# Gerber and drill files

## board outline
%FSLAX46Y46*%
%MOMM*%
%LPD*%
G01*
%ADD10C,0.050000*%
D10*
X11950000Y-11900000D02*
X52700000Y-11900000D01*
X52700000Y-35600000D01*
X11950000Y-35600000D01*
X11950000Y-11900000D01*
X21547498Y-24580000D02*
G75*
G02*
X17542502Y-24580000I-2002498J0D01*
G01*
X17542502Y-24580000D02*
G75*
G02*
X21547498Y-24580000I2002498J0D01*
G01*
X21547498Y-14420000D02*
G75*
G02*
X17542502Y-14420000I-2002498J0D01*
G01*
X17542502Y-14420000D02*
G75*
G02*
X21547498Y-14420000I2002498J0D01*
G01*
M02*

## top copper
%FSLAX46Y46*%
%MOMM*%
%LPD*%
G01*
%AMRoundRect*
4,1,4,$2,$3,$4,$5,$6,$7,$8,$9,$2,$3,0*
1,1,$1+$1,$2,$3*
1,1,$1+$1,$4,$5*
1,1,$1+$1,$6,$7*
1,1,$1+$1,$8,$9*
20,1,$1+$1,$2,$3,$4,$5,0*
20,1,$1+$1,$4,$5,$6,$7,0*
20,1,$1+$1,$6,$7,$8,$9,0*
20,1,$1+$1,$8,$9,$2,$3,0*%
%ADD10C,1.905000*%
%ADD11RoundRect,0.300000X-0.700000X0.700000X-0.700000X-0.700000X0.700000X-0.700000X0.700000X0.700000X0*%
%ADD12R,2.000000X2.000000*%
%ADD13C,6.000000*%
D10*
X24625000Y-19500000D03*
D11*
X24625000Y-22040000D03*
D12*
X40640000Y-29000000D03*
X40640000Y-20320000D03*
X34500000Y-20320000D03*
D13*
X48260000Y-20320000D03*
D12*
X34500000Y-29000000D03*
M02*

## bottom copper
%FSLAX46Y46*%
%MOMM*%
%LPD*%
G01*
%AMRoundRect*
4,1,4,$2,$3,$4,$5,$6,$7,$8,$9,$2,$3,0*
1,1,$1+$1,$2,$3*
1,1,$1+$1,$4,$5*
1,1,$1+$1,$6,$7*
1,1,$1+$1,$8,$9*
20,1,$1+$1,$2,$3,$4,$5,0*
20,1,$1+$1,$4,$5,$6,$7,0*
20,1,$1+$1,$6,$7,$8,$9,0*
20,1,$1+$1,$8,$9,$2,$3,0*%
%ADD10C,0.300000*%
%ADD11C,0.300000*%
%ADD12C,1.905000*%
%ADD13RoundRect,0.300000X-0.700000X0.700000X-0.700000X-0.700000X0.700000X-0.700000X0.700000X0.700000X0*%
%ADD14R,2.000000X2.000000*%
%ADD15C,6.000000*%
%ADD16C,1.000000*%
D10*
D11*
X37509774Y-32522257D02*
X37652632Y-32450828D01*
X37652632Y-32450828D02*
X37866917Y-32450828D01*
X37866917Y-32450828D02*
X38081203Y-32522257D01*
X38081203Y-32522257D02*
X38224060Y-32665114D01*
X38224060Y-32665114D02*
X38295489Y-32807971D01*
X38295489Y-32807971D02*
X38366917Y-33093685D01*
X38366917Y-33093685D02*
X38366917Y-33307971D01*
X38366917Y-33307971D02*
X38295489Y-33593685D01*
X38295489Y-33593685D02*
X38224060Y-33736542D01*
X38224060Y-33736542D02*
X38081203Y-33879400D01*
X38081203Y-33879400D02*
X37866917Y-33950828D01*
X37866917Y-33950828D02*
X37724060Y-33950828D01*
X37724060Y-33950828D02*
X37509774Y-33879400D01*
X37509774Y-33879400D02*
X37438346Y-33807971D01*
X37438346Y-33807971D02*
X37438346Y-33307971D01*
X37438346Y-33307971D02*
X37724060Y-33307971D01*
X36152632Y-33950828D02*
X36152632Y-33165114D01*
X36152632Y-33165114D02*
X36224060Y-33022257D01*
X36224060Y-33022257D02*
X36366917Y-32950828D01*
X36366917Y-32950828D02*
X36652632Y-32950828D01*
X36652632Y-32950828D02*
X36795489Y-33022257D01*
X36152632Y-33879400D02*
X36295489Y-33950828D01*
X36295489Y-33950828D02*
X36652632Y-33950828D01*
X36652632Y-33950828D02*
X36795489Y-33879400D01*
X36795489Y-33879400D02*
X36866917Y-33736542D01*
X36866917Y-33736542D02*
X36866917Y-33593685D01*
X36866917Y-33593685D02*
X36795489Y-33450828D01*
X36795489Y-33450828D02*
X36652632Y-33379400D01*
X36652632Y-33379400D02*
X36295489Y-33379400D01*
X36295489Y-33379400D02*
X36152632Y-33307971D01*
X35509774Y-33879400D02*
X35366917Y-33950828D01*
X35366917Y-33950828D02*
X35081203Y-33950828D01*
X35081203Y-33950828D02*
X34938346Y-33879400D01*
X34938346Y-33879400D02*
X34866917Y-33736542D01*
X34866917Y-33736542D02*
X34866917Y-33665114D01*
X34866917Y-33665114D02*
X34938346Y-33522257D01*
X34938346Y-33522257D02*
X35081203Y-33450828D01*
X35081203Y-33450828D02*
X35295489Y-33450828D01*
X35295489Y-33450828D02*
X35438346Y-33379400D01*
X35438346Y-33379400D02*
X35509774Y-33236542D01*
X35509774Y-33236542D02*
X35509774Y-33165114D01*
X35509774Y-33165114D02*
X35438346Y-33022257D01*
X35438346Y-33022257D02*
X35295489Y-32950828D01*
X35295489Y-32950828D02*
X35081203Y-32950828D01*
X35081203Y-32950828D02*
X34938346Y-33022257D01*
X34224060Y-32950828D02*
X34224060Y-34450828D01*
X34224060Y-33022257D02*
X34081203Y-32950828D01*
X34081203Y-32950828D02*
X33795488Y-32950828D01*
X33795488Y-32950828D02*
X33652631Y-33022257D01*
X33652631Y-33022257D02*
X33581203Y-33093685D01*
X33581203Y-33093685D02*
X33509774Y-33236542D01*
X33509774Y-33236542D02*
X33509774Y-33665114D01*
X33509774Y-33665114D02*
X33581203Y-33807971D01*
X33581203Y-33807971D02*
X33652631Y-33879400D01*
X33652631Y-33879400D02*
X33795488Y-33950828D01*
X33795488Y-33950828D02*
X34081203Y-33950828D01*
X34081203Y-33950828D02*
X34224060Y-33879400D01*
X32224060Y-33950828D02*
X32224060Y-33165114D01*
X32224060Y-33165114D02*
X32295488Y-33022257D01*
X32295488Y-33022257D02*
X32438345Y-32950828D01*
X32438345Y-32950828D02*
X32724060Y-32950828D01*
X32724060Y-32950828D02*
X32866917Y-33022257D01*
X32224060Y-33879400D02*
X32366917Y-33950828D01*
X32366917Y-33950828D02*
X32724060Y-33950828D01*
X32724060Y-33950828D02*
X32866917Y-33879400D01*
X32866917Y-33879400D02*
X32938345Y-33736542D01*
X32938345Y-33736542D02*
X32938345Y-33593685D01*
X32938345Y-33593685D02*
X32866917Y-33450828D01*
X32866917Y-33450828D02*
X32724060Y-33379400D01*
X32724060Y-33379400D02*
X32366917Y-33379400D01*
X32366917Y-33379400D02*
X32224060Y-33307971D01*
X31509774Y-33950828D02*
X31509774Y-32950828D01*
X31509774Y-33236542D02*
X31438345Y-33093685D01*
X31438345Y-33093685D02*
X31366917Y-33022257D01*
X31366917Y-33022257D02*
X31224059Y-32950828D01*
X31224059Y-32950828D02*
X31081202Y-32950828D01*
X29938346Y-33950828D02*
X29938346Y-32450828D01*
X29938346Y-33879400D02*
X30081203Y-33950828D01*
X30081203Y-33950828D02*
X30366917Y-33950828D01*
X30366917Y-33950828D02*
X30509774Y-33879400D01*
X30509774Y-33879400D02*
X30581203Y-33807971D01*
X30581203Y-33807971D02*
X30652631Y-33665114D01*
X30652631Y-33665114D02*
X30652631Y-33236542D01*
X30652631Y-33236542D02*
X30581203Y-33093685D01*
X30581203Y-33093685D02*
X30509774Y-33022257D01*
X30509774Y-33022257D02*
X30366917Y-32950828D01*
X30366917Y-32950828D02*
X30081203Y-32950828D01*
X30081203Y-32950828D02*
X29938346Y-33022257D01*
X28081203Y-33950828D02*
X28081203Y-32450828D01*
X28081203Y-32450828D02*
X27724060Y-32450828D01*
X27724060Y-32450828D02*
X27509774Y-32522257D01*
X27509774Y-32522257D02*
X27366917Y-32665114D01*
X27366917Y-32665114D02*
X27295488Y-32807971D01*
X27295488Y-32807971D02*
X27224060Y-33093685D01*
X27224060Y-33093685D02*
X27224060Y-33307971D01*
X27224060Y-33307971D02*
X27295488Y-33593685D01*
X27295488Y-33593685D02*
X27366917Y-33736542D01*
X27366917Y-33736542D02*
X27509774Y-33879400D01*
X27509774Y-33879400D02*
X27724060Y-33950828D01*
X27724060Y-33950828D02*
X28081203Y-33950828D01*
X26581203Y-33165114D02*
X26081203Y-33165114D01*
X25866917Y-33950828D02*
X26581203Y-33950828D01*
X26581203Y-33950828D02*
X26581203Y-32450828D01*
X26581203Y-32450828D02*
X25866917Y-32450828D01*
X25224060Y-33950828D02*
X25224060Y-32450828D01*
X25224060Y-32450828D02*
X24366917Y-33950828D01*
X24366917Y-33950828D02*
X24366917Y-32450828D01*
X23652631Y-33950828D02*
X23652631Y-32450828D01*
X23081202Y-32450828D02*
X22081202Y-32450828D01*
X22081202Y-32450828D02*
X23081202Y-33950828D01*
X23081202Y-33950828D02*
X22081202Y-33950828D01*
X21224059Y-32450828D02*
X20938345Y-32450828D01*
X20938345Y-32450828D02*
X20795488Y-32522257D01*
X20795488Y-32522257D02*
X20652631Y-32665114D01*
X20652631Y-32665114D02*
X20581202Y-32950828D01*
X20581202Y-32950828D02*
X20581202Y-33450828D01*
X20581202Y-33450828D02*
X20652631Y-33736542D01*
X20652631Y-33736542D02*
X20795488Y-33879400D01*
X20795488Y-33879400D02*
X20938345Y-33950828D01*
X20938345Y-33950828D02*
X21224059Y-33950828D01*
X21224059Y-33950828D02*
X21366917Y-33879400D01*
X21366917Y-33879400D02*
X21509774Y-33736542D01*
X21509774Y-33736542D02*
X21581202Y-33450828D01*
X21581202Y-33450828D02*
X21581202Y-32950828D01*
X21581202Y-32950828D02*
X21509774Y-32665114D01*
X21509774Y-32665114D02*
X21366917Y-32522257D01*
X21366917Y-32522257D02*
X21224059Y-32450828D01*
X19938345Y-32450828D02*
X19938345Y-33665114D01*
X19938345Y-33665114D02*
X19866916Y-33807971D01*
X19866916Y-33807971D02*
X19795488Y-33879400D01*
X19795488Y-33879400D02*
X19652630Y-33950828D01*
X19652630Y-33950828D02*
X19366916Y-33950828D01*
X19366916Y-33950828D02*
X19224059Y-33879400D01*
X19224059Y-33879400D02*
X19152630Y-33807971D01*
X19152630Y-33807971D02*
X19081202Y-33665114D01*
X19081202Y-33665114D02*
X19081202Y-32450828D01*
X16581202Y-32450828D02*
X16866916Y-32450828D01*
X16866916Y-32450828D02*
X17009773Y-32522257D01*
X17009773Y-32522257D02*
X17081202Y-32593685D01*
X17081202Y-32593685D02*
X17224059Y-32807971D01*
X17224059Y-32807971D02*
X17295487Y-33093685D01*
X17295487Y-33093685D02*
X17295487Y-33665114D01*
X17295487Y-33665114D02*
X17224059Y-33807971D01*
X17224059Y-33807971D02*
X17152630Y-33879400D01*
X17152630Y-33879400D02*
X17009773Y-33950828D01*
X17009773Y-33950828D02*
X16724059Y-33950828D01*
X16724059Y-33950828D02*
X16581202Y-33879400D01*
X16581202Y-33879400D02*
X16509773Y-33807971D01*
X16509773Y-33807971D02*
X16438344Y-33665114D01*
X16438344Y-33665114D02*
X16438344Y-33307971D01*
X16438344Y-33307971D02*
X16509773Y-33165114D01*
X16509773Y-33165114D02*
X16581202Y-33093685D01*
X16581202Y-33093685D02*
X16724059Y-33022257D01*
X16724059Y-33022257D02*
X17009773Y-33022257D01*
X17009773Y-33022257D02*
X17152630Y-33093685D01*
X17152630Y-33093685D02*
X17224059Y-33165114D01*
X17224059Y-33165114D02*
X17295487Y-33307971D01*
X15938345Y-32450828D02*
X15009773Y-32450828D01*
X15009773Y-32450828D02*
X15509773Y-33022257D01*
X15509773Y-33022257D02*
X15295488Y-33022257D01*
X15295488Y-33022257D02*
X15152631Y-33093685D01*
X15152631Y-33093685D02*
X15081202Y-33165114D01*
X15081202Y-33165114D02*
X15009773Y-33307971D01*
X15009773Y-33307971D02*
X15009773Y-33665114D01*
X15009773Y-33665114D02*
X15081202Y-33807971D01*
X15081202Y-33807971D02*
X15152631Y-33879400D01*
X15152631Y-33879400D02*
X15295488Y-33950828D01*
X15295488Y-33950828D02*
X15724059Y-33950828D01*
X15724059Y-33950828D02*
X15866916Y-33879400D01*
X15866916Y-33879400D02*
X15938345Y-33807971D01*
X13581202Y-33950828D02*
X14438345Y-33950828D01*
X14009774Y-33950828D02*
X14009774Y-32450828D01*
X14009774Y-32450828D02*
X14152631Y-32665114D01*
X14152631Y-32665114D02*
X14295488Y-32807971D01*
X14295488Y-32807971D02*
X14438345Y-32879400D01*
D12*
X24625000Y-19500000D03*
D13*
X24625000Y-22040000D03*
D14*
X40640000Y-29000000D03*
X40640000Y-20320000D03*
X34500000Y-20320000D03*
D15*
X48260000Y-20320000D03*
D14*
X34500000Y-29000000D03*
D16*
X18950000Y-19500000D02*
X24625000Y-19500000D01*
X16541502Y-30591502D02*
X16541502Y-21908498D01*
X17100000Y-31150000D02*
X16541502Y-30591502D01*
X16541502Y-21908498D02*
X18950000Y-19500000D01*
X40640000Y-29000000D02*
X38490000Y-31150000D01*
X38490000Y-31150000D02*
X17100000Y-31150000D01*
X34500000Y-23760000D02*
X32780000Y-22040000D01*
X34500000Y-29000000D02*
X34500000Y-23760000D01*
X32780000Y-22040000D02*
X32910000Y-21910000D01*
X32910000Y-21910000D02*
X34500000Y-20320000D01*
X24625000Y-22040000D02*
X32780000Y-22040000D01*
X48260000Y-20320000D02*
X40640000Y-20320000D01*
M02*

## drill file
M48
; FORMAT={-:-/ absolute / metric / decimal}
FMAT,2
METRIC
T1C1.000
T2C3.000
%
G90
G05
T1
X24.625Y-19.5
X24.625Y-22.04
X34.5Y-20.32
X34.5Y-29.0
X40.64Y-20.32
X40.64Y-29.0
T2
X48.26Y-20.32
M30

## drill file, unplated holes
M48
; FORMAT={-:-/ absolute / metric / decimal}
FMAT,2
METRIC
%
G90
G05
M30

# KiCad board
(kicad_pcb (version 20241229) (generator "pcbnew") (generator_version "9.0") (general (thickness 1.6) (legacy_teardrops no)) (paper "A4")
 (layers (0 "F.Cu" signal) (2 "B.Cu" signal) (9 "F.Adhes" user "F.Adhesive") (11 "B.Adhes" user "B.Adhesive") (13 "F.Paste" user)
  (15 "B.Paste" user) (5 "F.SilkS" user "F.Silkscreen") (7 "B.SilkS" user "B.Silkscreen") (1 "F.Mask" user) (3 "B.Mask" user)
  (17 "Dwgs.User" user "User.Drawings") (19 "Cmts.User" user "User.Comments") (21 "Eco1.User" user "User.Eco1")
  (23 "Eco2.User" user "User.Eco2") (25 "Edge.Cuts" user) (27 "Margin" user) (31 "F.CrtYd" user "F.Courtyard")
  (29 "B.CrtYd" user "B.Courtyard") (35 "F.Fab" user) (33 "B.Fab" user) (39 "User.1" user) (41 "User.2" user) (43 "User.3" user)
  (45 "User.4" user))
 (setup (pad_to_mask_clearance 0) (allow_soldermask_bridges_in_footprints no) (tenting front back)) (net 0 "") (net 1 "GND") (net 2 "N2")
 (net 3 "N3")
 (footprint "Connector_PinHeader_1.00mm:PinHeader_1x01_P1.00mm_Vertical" (layer "F.Cu") (at 40.64 29)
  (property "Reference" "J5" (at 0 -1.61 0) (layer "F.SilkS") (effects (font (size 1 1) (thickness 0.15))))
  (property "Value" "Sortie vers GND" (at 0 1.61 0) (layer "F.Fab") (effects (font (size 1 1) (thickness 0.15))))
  (pad "1" thru_hole rect (at 0 0) (size 2 2) (drill 1) (layers "*.Cu" "*.Mask") (remove_unused_layers no) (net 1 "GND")))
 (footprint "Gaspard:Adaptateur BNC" (layer "F.Cu") (at 31.625 16.96 -90)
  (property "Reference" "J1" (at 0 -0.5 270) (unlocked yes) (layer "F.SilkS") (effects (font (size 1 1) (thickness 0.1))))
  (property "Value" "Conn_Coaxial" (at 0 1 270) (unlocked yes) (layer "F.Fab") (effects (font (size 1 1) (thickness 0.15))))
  (fp_circle (center -2.54 12.08) (end -4.542498 12.08) (stroke (width 0.05) (type solid)) (fill no) (layer "Edge.Cuts"))
  (fp_circle (center 7.62 12.08) (end 5.617502 12.08) (stroke (width 0.05) (type solid)) (fill no) (layer "Edge.Cuts"))
  (pad "1" thru_hole roundrect (at 5.08 7 270) (size 2 2) (drill 1) (layers "*.Cu" "*.Mask") (remove_unused_layers no)
   (roundrect_rratio 0.15) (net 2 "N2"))
  (pad "2" thru_hole circle (at 2.54 7 270) (size 1.905 1.905) (drill 1) (layers "*.Cu" "*.Mask") (remove_unused_layers no) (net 1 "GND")))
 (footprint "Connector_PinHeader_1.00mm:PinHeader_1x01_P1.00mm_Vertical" (layer "F.Cu") (at 40.64 20.32)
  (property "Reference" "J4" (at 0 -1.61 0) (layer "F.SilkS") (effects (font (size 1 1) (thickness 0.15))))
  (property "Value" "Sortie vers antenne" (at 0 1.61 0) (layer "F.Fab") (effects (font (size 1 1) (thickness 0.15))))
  (pad "1" thru_hole rect (at 0 0) (size 2 2) (drill 1) (layers "*.Cu" "*.Mask") (remove_unused_layers no) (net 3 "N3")))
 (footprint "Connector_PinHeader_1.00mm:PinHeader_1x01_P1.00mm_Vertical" (layer "F.Cu") (at 34.5 20.32)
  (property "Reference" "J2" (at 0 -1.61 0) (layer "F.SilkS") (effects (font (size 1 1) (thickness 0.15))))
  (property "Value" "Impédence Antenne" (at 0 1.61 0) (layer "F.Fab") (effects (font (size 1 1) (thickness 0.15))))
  (pad "1" thru_hole rect (at 0 0) (size 2 2) (drill 1) (layers "*.Cu" "*.Mask") (remove_unused_layers no) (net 2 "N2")))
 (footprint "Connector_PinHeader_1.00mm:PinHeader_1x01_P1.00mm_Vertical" (layer "F.Cu") (at 48.26 20.32)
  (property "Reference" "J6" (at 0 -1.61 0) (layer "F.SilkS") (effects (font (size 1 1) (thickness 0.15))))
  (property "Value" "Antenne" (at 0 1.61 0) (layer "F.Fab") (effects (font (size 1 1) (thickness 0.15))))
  (pad "1" thru_hole circle (at 0 0) (size 6 6) (drill 3) (layers "*.Cu" "*.Mask") (remove_unused_layers no) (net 3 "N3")))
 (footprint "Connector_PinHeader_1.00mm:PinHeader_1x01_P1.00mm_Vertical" (layer "F.Cu") (at 34.5 29)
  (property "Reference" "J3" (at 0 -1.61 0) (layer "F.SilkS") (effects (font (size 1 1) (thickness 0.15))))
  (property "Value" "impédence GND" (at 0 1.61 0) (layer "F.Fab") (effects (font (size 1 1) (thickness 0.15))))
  (pad "1" thru_hole rect (at 0 0) (size 2 2) (drill 1) (layers "*.Cu" "*.Mask") (remove_unused_layers no) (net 2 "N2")))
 (gr_rect (start 11.95 11.9) (end 52.7 35.6) (stroke (width 0.05) (type solid)) (fill no) (layer "Edge.Cuts"))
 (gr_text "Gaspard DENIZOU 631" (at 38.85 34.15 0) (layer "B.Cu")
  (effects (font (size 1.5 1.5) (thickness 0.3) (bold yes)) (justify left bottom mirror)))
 (segment (start 34.5 23.76) (end 32.78 22.04) (width 1) (layer "B.Cu") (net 2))
 (segment (start 34.5 29) (end 34.5 23.76) (width 1) (layer "B.Cu") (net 2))
 (segment (start 32.78 22.04) (end 32.91 21.91) (width 1) (layer "B.Cu") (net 2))
 (segment (start 32.91 21.91) (end 34.5 20.32) (width 1) (layer "B.Cu") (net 2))
 (segment (start 24.625 22.04) (end 32.78 22.04) (width 1) (layer "B.Cu") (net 2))
 (segment (start 16.541502 30.591502) (end 16.541502 21.908498) (width 1) (layer "B.Cu") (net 1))
 (segment (start 17.1 31.15) (end 16.541502 30.591502) (width 1) (layer "B.Cu") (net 1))
 (segment (start 16.541502 21.908498) (end 18.95 19.5) (width 1) (layer "B.Cu") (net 1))
 (segment (start 40.64 29) (end 38.49 31.15) (width 1) (layer "B.Cu") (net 1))
 (segment (start 18.95 19.5) (end 24.625 19.5) (width 1) (layer "B.Cu") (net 1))
 (segment (start 38.49 31.15) (end 17.1 31.15) (width 1) (layer "B.Cu") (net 1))
 (segment (start 48.26 20.32) (end 40.64 20.32) (width 1) (layer "B.Cu") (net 3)))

